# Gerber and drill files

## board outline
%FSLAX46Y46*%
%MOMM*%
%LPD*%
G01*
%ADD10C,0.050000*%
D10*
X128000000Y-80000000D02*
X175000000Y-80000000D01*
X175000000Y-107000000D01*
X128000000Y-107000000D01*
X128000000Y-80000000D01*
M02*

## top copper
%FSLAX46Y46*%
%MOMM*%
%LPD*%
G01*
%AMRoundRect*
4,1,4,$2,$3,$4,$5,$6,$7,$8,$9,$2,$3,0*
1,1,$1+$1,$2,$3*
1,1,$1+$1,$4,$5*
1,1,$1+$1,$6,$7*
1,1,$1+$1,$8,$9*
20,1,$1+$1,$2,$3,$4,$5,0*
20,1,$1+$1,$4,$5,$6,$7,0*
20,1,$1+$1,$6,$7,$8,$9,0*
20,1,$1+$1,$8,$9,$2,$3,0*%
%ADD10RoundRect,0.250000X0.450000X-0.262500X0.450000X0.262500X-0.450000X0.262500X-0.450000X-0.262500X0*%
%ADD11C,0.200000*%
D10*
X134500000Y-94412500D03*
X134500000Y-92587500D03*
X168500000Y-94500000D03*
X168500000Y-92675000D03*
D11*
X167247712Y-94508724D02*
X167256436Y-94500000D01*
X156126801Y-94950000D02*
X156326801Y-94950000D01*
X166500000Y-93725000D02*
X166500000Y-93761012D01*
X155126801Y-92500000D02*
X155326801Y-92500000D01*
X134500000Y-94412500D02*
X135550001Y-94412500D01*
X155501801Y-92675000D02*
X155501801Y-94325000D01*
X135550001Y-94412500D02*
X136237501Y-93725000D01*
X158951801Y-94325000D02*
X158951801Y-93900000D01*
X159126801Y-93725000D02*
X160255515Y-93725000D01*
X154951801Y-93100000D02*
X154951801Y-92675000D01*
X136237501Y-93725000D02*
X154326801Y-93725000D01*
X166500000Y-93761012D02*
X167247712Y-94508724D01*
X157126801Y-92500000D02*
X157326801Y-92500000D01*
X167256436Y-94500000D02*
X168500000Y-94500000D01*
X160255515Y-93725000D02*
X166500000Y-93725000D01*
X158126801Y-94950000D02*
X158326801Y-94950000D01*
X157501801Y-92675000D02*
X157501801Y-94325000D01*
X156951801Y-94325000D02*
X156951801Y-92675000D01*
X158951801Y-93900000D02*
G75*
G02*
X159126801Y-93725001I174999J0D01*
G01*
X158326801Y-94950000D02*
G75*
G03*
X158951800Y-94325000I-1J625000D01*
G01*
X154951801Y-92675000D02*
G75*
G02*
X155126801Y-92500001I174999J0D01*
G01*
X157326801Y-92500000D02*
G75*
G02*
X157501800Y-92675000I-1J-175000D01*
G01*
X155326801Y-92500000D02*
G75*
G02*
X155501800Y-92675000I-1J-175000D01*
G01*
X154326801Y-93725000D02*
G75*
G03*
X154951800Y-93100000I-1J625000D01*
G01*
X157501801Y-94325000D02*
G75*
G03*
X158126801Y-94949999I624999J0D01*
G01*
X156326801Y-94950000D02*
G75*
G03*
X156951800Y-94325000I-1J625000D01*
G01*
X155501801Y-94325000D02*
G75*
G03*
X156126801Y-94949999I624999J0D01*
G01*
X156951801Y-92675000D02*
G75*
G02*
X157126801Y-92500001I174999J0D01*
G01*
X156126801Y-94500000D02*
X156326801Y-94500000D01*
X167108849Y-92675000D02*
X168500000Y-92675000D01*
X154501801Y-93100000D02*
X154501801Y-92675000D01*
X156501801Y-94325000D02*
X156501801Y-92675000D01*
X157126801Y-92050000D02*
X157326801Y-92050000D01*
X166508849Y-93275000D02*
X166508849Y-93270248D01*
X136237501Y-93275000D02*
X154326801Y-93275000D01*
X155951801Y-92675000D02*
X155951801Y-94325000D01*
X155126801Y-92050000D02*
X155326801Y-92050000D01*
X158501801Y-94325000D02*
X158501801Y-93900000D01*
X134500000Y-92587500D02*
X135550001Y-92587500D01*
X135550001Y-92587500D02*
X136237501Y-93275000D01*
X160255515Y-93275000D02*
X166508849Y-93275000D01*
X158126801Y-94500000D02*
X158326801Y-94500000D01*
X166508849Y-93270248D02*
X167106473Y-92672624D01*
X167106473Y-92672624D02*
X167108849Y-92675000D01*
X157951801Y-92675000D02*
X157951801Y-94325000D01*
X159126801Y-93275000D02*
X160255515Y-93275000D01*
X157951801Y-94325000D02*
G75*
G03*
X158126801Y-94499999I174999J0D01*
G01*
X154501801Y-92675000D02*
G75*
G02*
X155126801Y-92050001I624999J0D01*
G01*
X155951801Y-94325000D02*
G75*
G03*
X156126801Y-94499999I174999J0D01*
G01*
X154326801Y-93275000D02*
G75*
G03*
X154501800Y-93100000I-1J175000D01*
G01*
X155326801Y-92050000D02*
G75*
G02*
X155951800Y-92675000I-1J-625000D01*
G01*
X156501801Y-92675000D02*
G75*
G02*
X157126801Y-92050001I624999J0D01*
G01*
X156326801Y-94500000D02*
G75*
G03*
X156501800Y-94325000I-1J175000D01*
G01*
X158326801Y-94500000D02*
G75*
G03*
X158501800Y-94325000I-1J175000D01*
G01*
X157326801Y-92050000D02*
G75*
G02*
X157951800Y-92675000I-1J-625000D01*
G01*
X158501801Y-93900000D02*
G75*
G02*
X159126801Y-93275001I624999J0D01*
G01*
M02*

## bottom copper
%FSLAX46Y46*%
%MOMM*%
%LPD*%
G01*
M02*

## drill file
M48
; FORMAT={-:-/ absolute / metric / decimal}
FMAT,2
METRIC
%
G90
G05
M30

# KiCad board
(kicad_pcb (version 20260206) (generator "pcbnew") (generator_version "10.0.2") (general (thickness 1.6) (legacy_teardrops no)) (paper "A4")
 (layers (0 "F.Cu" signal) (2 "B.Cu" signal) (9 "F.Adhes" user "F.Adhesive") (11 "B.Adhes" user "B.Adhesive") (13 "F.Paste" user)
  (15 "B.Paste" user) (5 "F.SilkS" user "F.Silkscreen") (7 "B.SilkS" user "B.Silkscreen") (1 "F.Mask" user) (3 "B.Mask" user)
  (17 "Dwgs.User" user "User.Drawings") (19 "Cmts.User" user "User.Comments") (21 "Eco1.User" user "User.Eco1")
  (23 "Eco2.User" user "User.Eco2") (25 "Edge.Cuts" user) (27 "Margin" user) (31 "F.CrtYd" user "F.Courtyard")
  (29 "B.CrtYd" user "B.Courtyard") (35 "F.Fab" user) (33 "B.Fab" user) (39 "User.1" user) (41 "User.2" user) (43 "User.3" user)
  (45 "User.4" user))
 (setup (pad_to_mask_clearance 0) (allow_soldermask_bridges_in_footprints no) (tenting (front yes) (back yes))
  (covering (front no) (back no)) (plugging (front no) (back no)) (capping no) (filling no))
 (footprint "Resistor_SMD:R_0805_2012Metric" (layer "F.Cu") (at 134.5 93.5 90)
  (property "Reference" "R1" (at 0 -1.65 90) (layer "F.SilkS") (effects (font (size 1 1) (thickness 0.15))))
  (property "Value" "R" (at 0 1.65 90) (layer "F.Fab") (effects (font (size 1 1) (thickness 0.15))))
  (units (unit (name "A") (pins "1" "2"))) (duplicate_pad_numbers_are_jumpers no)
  (pad "1" smd roundrect (at -0.9125 0 90) (size 1.025 1.4) (layers "F.Cu" "F.Mask" "F.Paste") (roundrect_rratio 0.243902) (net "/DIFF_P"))
  (pad "2" smd roundrect (at 0.9125 0 90) (size 1.025 1.4) (layers "F.Cu" "F.Mask" "F.Paste") (roundrect_rratio 0.243902) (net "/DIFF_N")))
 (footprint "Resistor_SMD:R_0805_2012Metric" (layer "F.Cu") (at 168.5 93.5875 90)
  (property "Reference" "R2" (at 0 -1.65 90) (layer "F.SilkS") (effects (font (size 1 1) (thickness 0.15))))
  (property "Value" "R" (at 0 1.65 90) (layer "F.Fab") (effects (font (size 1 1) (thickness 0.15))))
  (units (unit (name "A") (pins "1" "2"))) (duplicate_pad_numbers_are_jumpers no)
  (pad "1" smd roundrect (at -0.9125 0 90) (size 1.025 1.4) (layers "F.Cu" "F.Mask" "F.Paste") (roundrect_rratio 0.243902) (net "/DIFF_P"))
  (pad "2" smd roundrect (at 0.9125 0 90) (size 1.025 1.4) (layers "F.Cu" "F.Mask" "F.Paste") (roundrect_rratio 0.243902) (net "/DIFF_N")))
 (gr_rect (start 128 80) (end 175 107) (stroke (width 0.05) (type default)) (fill no) (layer "Edge.Cuts"))
 (segment (start 167.247712 94.508724) (end 167.256436 94.5) (width 0.2) (layer "F.Cu") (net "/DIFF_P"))
 (segment (start 156.126801 94.95) (end 156.326801 94.95) (width 0.2) (layer "F.Cu") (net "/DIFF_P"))
 (segment (start 166.5 93.725) (end 166.5 93.761012) (width 0.2) (layer "F.Cu") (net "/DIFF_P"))
 (segment (start 155.126801 92.5) (end 155.326801 92.5) (width 0.2) (layer "F.Cu") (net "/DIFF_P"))
 (segment (start 134.5 94.4125) (end 135.550001 94.4125) (width 0.2) (layer "F.Cu") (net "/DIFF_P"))
 (segment (start 155.501801 92.675) (end 155.501801 94.325) (width 0.2) (layer "F.Cu") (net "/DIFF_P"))
 (segment (start 135.550001 94.4125) (end 136.237501 93.725) (width 0.2) (layer "F.Cu") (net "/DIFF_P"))
 (segment (start 158.951801 94.325) (end 158.951801 93.9) (width 0.2) (layer "F.Cu") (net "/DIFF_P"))
 (segment (start 159.126801 93.725) (end 160.255515 93.725) (width 0.2) (layer "F.Cu") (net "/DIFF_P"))
 (segment (start 154.951801 93.1) (end 154.951801 92.675) (width 0.2) (layer "F.Cu") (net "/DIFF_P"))
 (segment (start 136.237501 93.725) (end 154.326801 93.725) (width 0.2) (layer "F.Cu") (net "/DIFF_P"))
 (segment (start 166.5 93.761012) (end 167.247712 94.508724) (width 0.2) (layer "F.Cu") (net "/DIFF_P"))
 (segment (start 157.126801 92.5) (end 157.326801 92.5) (width 0.2) (layer "F.Cu") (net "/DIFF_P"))
 (segment (start 167.256436 94.5) (end 168.5 94.5) (width 0.2) (layer "F.Cu") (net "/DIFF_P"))
 (segment (start 160.255515 93.725) (end 166.5 93.725) (width 0.2) (layer "F.Cu") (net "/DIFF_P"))
 (segment (start 158.126801 94.95) (end 158.326801 94.95) (width 0.2) (layer "F.Cu") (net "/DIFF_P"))
 (segment (start 157.501801 92.675) (end 157.501801 94.325) (width 0.2) (layer "F.Cu") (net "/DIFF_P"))
 (segment (start 156.951801 94.325) (end 156.951801 92.675) (width 0.2) (layer "F.Cu") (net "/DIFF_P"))
 (arc (start 158.951801 93.9) (mid 159.003057 93.776256) (end 159.126801 93.725) (width 0.2) (layer "F.Cu") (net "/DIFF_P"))
 (arc (start 158.326801 94.95) (mid 158.768743 94.766942) (end 158.951801 94.325) (width 0.2) (layer "F.Cu") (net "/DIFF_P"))
 (arc (start 154.951801 92.675) (mid 155.003057 92.551256) (end 155.126801 92.5) (width 0.2) (layer "F.Cu") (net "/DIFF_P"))
 (arc (start 157.326801 92.5) (mid 157.450545 92.551256) (end 157.501801 92.675) (width 0.2) (layer "F.Cu") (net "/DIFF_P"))
 (arc (start 155.326801 92.5) (mid 155.450545 92.551256) (end 155.501801 92.675) (width 0.2) (layer "F.Cu") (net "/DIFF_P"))
 (arc (start 154.326801 93.725) (mid 154.768743 93.541942) (end 154.951801 93.1) (width 0.2) (layer "F.Cu") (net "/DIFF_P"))
 (arc (start 157.501801 94.325) (mid 157.684859 94.766942) (end 158.126801 94.95) (width 0.2) (layer "F.Cu") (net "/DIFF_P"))
 (arc (start 156.326801 94.95) (mid 156.768743 94.766942) (end 156.951801 94.325) (width 0.2) (layer "F.Cu") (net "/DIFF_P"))
 (arc (start 155.501801 94.325) (mid 155.684859 94.766942) (end 156.126801 94.95) (width 0.2) (layer "F.Cu") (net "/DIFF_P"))
 (arc (start 156.951801 92.675) (mid 157.003057 92.551256) (end 157.126801 92.5) (width 0.2) (layer "F.Cu") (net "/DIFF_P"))
 (segment (start 156.126801 94.5) (end 156.326801 94.5) (width 0.2) (layer "F.Cu") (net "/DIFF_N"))
 (segment (start 167.108849 92.675) (end 168.5 92.675) (width 0.2) (layer "F.Cu") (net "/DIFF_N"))
 (segment (start 154.501801 93.1) (end 154.501801 92.675) (width 0.2) (layer "F.Cu") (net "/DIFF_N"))
 (segment (start 156.501801 94.325) (end 156.501801 92.675) (width 0.2) (layer "F.Cu") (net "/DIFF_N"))
 (segment (start 157.126801 92.05) (end 157.326801 92.05) (width 0.2) (layer "F.Cu") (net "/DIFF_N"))
 (segment (start 166.508849 93.275) (end 166.508849 93.270248) (width 0.2) (layer "F.Cu") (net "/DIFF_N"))
 (segment (start 136.237501 93.275) (end 154.326801 93.275) (width 0.2) (layer "F.Cu") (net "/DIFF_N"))
 (segment (start 155.951801 92.675) (end 155.951801 94.325) (width 0.2) (layer "F.Cu") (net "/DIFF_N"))
 (segment (start 155.126801 92.05) (end 155.326801 92.05) (width 0.2) (layer "F.Cu") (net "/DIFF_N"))
 (segment (start 158.501801 94.325) (end 158.501801 93.9) (width 0.2) (layer "F.Cu") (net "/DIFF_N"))
 (segment (start 134.5 92.5875) (end 135.550001 92.5875) (width 0.2) (layer "F.Cu") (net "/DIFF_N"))
 (segment (start 135.550001 92.5875) (end 136.237501 93.275) (width 0.2) (layer "F.Cu") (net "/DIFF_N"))
 (segment (start 160.255515 93.275) (end 166.508849 93.275) (width 0.2) (layer "F.Cu") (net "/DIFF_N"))
 (segment (start 158.126801 94.5) (end 158.326801 94.5) (width 0.2) (layer "F.Cu") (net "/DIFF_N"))
 (segment (start 166.508849 93.270248) (end 167.106473 92.672624) (width 0.2) (layer "F.Cu") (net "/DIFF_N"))
 (segment (start 167.106473 92.672624) (end 167.108849 92.675) (width 0.2) (layer "F.Cu") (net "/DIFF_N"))
 (segment (start 157.951801 92.675) (end 157.951801 94.325) (width 0.2) (layer "F.Cu") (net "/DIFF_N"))
 (segment (start 159.126801 93.275) (end 160.255515 93.275) (width 0.2) (layer "F.Cu") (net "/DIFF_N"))
 (arc (start 157.951801 94.325) (mid 158.003057 94.448744) (end 158.126801 94.5) (width 0.2) (layer "F.Cu") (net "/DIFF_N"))
 (arc (start 154.501801 92.675) (mid 154.684859 92.233058) (end 155.126801 92.05) (width 0.2) (layer "F.Cu") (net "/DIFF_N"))
 (arc (start 155.951801 94.325) (mid 156.003057 94.448744) (end 156.126801 94.5) (width 0.2) (layer "F.Cu") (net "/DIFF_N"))
 (arc (start 154.326801 93.275) (mid 154.450545 93.223744) (end 154.501801 93.1) (width 0.2) (layer "F.Cu") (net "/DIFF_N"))
 (arc (start 155.326801 92.05) (mid 155.768743 92.233058) (end 155.951801 92.675) (width 0.2) (layer "F.Cu") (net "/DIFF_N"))
 (arc (start 156.501801 92.675) (mid 156.684859 92.233058) (end 157.126801 92.05) (width 0.2) (layer "F.Cu") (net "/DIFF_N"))
 (arc (start 156.326801 94.5) (mid 156.450545 94.448744) (end 156.501801 94.325) (width 0.2) (layer "F.Cu") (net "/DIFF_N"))
 (arc (start 158.326801 94.5) (mid 158.450545 94.448744) (end 158.501801 94.325) (width 0.2) (layer "F.Cu") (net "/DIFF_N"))
 (arc (start 157.326801 92.05) (mid 157.768743 92.233058) (end 157.951801 92.675) (width 0.2) (layer "F.Cu") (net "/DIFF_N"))
 (arc (start 158.501801 93.9) (mid 158.684859 93.458058) (end 159.126801 93.275) (width 0.2) (layer "F.Cu") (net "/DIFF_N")))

